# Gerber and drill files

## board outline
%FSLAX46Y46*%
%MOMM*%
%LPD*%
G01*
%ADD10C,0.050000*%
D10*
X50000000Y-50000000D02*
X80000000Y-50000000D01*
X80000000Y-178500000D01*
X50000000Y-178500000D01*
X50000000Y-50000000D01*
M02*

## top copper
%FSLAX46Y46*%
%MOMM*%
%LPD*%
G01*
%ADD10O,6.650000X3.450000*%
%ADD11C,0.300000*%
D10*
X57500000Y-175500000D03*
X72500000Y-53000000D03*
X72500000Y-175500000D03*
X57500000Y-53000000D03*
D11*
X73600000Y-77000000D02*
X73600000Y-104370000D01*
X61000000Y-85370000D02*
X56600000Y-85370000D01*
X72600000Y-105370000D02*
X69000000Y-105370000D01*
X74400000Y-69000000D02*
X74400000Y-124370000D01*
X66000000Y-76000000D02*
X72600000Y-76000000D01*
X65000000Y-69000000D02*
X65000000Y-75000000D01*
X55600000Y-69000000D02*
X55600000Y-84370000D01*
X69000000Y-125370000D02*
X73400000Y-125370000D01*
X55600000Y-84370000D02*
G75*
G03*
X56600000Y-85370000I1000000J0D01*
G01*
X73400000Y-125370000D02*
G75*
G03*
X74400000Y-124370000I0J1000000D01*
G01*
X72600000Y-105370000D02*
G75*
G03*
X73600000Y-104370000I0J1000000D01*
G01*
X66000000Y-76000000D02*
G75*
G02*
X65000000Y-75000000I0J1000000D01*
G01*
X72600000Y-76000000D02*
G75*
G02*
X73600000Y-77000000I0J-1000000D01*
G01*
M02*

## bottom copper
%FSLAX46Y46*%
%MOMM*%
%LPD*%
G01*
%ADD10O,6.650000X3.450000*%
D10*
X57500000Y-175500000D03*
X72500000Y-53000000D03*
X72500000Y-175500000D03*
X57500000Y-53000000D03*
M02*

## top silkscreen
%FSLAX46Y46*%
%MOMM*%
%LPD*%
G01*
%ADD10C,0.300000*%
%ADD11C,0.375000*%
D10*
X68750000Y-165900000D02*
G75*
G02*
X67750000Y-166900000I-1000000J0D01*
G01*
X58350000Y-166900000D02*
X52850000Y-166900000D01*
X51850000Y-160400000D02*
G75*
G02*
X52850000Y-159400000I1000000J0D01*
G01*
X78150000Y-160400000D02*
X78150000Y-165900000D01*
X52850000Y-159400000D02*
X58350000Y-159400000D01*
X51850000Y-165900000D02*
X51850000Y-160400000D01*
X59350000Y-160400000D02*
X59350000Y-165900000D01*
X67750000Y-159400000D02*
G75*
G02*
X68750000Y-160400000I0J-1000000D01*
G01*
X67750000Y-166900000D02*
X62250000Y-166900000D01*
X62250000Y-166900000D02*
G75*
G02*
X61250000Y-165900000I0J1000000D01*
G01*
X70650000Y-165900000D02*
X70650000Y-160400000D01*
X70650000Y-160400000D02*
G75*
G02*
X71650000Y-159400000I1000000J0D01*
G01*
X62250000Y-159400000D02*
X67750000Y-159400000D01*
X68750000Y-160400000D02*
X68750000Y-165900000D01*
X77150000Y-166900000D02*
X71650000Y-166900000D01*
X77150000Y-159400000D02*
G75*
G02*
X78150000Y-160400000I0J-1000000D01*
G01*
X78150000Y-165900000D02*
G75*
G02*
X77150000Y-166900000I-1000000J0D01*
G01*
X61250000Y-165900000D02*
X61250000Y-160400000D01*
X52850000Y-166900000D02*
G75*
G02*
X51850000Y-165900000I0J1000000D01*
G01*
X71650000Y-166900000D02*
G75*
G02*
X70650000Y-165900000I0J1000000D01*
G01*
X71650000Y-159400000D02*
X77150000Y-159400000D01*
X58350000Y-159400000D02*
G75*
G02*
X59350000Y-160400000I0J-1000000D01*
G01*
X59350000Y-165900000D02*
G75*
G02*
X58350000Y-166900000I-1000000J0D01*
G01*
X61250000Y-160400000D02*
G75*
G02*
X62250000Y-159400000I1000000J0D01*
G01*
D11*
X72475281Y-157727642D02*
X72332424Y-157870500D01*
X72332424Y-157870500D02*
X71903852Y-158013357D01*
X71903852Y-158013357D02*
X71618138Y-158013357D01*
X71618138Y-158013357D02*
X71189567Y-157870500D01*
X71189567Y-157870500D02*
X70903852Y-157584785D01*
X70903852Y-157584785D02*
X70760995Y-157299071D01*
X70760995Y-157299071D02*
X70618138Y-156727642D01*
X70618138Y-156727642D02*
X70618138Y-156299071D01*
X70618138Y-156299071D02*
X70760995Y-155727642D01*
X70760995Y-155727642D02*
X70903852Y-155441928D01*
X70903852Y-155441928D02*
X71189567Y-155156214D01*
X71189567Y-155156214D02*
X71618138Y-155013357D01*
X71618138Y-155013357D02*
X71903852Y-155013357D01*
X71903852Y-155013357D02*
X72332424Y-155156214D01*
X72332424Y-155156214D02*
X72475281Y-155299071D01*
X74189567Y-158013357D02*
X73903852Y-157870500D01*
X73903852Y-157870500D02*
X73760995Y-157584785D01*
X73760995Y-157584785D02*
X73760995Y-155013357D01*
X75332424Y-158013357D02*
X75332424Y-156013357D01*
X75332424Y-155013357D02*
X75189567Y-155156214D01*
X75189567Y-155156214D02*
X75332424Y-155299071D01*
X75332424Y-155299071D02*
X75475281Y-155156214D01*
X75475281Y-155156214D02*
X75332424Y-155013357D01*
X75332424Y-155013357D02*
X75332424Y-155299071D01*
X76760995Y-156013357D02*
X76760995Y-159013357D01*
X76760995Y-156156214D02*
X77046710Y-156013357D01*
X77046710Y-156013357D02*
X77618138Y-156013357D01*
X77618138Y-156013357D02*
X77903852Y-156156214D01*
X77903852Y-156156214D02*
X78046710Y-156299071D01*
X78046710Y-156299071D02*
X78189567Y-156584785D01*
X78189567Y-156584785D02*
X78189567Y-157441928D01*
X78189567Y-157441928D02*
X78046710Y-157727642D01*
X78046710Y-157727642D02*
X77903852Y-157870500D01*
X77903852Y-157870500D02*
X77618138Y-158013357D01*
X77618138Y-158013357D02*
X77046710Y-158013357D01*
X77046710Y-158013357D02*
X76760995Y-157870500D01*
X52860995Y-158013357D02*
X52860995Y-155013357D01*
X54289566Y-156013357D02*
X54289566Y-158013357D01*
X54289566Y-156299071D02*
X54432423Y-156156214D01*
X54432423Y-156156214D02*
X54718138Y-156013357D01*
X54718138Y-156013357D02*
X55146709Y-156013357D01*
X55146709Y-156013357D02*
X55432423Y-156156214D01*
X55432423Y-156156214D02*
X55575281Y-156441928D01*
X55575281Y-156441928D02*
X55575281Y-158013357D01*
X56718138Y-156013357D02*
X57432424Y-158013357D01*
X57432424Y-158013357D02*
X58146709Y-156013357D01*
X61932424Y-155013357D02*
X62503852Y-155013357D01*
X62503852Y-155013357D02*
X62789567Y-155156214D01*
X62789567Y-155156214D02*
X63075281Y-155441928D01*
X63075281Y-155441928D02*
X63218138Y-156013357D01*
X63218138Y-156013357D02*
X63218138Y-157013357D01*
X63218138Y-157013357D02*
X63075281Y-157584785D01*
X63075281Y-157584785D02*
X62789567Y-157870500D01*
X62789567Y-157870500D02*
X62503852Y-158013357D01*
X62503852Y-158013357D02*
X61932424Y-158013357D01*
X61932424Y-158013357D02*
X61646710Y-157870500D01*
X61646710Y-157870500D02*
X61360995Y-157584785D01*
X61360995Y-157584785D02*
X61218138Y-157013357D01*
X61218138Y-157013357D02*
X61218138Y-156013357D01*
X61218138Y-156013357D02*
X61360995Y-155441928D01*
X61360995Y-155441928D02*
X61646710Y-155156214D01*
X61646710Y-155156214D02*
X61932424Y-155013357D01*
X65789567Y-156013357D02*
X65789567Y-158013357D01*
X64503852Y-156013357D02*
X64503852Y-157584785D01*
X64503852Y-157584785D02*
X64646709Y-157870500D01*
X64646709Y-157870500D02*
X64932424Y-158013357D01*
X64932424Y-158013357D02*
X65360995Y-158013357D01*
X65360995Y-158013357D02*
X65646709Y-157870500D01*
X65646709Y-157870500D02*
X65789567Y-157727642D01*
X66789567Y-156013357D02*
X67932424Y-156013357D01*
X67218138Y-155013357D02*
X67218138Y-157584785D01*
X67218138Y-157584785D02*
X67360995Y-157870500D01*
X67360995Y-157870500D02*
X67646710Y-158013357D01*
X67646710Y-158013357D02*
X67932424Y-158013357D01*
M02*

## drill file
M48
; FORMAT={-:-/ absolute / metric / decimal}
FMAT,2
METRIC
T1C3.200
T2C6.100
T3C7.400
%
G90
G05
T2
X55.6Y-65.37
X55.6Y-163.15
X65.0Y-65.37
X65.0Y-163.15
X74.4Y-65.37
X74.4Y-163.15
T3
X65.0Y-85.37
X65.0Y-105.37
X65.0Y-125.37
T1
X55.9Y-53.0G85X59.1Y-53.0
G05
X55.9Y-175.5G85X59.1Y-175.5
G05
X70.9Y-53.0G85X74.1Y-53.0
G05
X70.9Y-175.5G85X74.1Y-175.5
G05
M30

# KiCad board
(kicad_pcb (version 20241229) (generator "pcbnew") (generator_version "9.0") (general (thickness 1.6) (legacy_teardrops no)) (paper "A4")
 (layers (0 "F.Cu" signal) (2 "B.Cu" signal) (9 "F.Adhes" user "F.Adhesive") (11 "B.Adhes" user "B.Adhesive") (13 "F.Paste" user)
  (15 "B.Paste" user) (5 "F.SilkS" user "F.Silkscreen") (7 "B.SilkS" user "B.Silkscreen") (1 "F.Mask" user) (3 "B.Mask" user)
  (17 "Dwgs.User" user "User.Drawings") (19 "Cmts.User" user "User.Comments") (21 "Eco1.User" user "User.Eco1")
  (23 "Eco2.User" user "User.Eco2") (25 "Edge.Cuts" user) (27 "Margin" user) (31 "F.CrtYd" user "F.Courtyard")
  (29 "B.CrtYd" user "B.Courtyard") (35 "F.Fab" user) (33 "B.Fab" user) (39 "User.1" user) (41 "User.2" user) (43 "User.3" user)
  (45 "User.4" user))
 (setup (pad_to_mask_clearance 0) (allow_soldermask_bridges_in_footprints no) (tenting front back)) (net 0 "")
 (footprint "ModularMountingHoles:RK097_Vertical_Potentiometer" (layer "F.Cu") (at 65 125.37)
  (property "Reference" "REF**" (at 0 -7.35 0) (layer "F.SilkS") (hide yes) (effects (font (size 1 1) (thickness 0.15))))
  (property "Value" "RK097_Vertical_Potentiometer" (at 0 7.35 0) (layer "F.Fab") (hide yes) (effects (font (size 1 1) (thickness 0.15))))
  (pad "" np_thru_hole circle (at 0 0) (size 7.4 7.4) (drill 7.4) (layers "*.Cu" "*.Mask")))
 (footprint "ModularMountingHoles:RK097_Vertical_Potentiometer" (layer "F.Cu") (at 65 85.37)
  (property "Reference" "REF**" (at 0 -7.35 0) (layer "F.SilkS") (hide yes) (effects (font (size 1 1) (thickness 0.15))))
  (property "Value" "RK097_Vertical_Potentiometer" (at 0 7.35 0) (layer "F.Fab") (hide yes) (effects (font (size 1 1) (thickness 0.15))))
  (pad "" np_thru_hole circle (at 0 0) (size 7.4 7.4) (drill 7.4) (layers "*.Cu" "*.Mask")))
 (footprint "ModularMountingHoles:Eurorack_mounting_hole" (layer "F.Cu") (at 57.5 175.5)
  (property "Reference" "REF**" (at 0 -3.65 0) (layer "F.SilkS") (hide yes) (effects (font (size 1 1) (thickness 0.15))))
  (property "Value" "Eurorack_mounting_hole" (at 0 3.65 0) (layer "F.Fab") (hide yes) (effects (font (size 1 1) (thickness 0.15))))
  (pad "1" thru_hole oval (at 0 0) (size 6.65 3.45) (drill oval 6.4 3.2) (layers "*.Cu" "*.Mask") (remove_unused_layers no) (zone_connect 2)))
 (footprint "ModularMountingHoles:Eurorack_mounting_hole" (layer "F.Cu") (at 72.5 53)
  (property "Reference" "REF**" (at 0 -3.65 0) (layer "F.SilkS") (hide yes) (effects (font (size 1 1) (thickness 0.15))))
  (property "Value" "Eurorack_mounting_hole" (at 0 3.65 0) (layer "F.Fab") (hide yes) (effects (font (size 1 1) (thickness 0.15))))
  (pad "1" thru_hole oval (at 0 0) (size 6.65 3.45) (drill oval 6.4 3.2) (layers "*.Cu" "*.Mask") (remove_unused_layers no) (zone_connect 2)))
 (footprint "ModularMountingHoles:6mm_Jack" (layer "F.Cu") (at 55.6 65.37)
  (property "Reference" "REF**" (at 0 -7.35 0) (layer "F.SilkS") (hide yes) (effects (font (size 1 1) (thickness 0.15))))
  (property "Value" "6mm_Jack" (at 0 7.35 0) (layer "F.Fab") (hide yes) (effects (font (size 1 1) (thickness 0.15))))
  (pad "" np_thru_hole circle (at 0 0) (size 6.1 6.1) (drill 6.1) (layers "*.Cu" "*.Mask")))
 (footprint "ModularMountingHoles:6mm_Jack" (layer "F.Cu") (at 74.4 65.37)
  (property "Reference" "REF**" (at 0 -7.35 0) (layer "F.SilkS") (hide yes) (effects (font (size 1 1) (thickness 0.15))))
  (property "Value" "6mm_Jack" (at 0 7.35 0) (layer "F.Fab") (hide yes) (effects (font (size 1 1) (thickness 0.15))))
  (pad "" np_thru_hole circle (at 0 0) (size 6.1 6.1) (drill 6.1) (layers "*.Cu" "*.Mask")))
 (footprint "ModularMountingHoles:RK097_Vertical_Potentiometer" (layer "F.Cu") (at 65 105.37)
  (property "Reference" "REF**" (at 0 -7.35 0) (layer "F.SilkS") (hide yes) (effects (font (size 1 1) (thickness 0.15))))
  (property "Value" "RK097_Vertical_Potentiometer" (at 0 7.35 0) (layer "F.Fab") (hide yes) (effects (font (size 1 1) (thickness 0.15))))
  (pad "" np_thru_hole circle (at 0 0) (size 7.4 7.4) (drill 7.4) (layers "*.Cu" "*.Mask")))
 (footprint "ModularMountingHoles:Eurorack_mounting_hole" (layer "F.Cu") (at 72.5 175.5)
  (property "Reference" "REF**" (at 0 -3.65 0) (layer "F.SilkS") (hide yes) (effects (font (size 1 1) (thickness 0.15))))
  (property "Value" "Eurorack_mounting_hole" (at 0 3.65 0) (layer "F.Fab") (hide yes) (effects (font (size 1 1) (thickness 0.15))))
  (pad "1" thru_hole oval (at 0 0) (size 6.65 3.45) (drill oval 6.4 3.2) (layers "*.Cu" "*.Mask") (remove_unused_layers no) (zone_connect 2)))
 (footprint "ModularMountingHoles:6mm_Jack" (layer "F.Cu") (at 74.4 163.15)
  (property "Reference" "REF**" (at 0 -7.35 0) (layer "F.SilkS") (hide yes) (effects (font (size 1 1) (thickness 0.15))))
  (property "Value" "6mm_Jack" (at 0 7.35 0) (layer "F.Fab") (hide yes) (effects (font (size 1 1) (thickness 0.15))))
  (pad "" np_thru_hole circle (at 0 0) (size 6.1 6.1) (drill 6.1) (layers "*.Cu" "*.Mask")))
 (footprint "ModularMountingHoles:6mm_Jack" (layer "F.Cu") (at 55.6 163.15)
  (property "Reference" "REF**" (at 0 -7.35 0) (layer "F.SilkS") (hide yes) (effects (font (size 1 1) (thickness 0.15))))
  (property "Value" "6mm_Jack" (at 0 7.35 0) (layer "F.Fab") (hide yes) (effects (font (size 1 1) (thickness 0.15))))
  (pad "" np_thru_hole circle (at 0 0) (size 6.1 6.1) (drill 6.1) (layers "*.Cu" "*.Mask")))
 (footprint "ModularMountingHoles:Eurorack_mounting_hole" (layer "F.Cu") (at 57.5 53)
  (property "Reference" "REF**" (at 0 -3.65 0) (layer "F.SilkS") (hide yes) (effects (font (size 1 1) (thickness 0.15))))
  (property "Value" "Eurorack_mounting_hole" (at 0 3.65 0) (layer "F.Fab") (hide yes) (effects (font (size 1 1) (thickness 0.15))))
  (pad "1" thru_hole oval (at 0 0) (size 6.65 3.45) (drill oval 6.4 3.2) (layers "*.Cu" "*.Mask") (remove_unused_layers no) (zone_connect 2)))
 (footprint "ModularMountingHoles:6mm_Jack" (layer "F.Cu") (at 65 163.15)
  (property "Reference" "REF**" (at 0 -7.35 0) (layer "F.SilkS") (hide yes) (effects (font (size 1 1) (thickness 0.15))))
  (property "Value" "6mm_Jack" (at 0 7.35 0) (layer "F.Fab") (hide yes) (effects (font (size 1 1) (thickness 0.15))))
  (pad "" np_thru_hole circle (at 0 0) (size 6.1 6.1) (drill 6.1) (layers "*.Cu" "*.Mask")))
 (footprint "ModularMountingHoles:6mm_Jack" (layer "F.Cu") (at 65 65.37)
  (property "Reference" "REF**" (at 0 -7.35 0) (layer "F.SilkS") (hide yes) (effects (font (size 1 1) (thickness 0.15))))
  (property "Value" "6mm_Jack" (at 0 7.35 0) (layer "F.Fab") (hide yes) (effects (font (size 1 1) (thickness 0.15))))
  (pad "" np_thru_hole circle (at 0 0) (size 6.1 6.1) (drill 6.1) (layers "*.Cu" "*.Mask")))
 (gr_arc (start 68.75 165.9) (mid 68.457107 166.607107) (end 67.75 166.9) (stroke (width 0.3) (type default)) (layer "F.SilkS"))
 (gr_line (start 58.35 166.9) (end 52.85 166.9) (stroke (width 0.3) (type default)) (layer "F.SilkS"))
 (gr_arc (start 51.85 160.4) (mid 52.142893 159.692893) (end 52.85 159.4) (stroke (width 0.3) (type default)) (layer "F.SilkS"))
 (gr_line (start 78.15 160.4) (end 78.15 165.9) (stroke (width 0.3) (type default)) (layer "F.SilkS"))
 (gr_line (start 52.85 159.4) (end 58.35 159.4) (stroke (width 0.3) (type default)) (layer "F.SilkS"))
 (gr_line (start 51.85 165.9) (end 51.85 160.4) (stroke (width 0.3) (type default)) (layer "F.SilkS"))
 (gr_line (start 59.35 160.4) (end 59.35 165.9) (stroke (width 0.3) (type default)) (layer "F.SilkS"))
 (gr_arc (start 67.75 159.4) (mid 68.457107 159.692893) (end 68.75 160.4) (stroke (width 0.3) (type default)) (layer "F.SilkS"))
 (gr_line (start 67.75 166.9) (end 62.25 166.9) (stroke (width 0.3) (type default)) (layer "F.SilkS"))
 (gr_arc (start 62.25 166.9) (mid 61.542893 166.607107) (end 61.25 165.9) (stroke (width 0.3) (type default)) (layer "F.SilkS"))
 (gr_line (start 70.65 165.9) (end 70.65 160.4) (stroke (width 0.3) (type default)) (layer "F.SilkS"))
 (gr_arc (start 70.65 160.4) (mid 70.942893 159.692893) (end 71.65 159.4) (stroke (width 0.3) (type default)) (layer "F.SilkS"))
 (gr_line (start 62.25 159.4) (end 67.75 159.4) (stroke (width 0.3) (type default)) (layer "F.SilkS"))
 (gr_line (start 68.75 160.4) (end 68.75 165.9) (stroke (width 0.3) (type default)) (layer "F.SilkS"))
 (gr_line (start 77.15 166.9) (end 71.65 166.9) (stroke (width 0.3) (type default)) (layer "F.SilkS"))
 (gr_arc (start 77.15 159.4) (mid 77.857107 159.692893) (end 78.15 160.4) (stroke (width 0.3) (type default)) (layer "F.SilkS"))
 (gr_arc (start 78.15 165.9) (mid 77.857107 166.607107) (end 77.15 166.9) (stroke (width 0.3) (type default)) (layer "F.SilkS"))
 (gr_line (start 61.25 165.9) (end 61.25 160.4) (stroke (width 0.3) (type default)) (layer "F.SilkS"))
 (gr_arc (start 52.85 166.9) (mid 52.142893 166.607107) (end 51.85 165.9) (stroke (width 0.3) (type default)) (layer "F.SilkS"))
 (gr_arc (start 71.65 166.9) (mid 70.942893 166.607107) (end 70.65 165.9) (stroke (width 0.3) (type default)) (layer "F.SilkS"))
 (gr_line (start 71.65 159.4) (end 77.15 159.4) (stroke (width 0.3) (type default)) (layer "F.SilkS"))
 (gr_arc (start 58.35 159.4) (mid 59.057107 159.692893) (end 59.35 160.4) (stroke (width 0.3) (type default)) (layer "F.SilkS"))
 (gr_arc (start 59.35 165.9) (mid 59.057107 166.607107) (end 58.35 166.9) (stroke (width 0.3) (type default)) (layer "F.SilkS"))
 (gr_arc (start 61.25 160.4) (mid 61.542893 159.692893) (end 62.25 159.4) (stroke (width 0.3) (type default)) (layer "F.SilkS"))
 (gr_rect (start 50 50) (end 80 178.5) (stroke (width 0.05) (type solid)) (fill no) (layer "Edge.Cuts"))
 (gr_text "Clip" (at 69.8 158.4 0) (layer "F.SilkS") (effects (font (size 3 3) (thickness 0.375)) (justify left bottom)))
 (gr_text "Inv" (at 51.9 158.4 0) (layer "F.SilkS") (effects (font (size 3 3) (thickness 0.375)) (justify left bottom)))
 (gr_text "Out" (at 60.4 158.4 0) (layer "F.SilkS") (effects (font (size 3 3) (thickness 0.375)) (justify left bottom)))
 (segment (start 73.6 77) (end 73.6 104.37) (width 0.3) (layer "F.Cu") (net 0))
 (segment (start 61 85.37) (end 56.6 85.37) (width 0.3) (layer "F.Cu") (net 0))
 (segment (start 72.6 105.37) (end 69 105.37) (width 0.3) (layer "F.Cu") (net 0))
 (segment (start 74.4 69) (end 74.4 124.37) (width 0.3) (layer "F.Cu") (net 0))
 (segment (start 66 76) (end 72.6 76) (width 0.3) (layer "F.Cu") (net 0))
 (segment (start 65 69) (end 65 75) (width 0.3) (layer "F.Cu") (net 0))
 (segment (start 55.6 69) (end 55.6 84.37) (width 0.3) (layer "F.Cu") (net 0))
 (segment (start 69 125.37) (end 73.4 125.37) (width 0.3) (layer "F.Cu") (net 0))
 (arc (start 55.6 84.37) (mid 55.892893 85.077107) (end 56.6 85.37) (width 0.3) (layer "F.Cu") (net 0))
 (arc (start 73.4 125.37) (mid 74.107107 125.077107) (end 74.4 124.37) (width 0.3) (layer "F.Cu") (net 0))
 (arc (start 72.6 105.37) (mid 73.307107 105.077107) (end 73.6 104.37) (width 0.3) (layer "F.Cu") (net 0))
 (arc (start 66 76) (mid 65.292893 75.707107) (end 65 75) (width 0.3) (layer "F.Cu") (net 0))
 (arc (start 72.6 76) (mid 73.307107 76.292893) (end 73.6 77) (width 0.3) (layer "F.Cu") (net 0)))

